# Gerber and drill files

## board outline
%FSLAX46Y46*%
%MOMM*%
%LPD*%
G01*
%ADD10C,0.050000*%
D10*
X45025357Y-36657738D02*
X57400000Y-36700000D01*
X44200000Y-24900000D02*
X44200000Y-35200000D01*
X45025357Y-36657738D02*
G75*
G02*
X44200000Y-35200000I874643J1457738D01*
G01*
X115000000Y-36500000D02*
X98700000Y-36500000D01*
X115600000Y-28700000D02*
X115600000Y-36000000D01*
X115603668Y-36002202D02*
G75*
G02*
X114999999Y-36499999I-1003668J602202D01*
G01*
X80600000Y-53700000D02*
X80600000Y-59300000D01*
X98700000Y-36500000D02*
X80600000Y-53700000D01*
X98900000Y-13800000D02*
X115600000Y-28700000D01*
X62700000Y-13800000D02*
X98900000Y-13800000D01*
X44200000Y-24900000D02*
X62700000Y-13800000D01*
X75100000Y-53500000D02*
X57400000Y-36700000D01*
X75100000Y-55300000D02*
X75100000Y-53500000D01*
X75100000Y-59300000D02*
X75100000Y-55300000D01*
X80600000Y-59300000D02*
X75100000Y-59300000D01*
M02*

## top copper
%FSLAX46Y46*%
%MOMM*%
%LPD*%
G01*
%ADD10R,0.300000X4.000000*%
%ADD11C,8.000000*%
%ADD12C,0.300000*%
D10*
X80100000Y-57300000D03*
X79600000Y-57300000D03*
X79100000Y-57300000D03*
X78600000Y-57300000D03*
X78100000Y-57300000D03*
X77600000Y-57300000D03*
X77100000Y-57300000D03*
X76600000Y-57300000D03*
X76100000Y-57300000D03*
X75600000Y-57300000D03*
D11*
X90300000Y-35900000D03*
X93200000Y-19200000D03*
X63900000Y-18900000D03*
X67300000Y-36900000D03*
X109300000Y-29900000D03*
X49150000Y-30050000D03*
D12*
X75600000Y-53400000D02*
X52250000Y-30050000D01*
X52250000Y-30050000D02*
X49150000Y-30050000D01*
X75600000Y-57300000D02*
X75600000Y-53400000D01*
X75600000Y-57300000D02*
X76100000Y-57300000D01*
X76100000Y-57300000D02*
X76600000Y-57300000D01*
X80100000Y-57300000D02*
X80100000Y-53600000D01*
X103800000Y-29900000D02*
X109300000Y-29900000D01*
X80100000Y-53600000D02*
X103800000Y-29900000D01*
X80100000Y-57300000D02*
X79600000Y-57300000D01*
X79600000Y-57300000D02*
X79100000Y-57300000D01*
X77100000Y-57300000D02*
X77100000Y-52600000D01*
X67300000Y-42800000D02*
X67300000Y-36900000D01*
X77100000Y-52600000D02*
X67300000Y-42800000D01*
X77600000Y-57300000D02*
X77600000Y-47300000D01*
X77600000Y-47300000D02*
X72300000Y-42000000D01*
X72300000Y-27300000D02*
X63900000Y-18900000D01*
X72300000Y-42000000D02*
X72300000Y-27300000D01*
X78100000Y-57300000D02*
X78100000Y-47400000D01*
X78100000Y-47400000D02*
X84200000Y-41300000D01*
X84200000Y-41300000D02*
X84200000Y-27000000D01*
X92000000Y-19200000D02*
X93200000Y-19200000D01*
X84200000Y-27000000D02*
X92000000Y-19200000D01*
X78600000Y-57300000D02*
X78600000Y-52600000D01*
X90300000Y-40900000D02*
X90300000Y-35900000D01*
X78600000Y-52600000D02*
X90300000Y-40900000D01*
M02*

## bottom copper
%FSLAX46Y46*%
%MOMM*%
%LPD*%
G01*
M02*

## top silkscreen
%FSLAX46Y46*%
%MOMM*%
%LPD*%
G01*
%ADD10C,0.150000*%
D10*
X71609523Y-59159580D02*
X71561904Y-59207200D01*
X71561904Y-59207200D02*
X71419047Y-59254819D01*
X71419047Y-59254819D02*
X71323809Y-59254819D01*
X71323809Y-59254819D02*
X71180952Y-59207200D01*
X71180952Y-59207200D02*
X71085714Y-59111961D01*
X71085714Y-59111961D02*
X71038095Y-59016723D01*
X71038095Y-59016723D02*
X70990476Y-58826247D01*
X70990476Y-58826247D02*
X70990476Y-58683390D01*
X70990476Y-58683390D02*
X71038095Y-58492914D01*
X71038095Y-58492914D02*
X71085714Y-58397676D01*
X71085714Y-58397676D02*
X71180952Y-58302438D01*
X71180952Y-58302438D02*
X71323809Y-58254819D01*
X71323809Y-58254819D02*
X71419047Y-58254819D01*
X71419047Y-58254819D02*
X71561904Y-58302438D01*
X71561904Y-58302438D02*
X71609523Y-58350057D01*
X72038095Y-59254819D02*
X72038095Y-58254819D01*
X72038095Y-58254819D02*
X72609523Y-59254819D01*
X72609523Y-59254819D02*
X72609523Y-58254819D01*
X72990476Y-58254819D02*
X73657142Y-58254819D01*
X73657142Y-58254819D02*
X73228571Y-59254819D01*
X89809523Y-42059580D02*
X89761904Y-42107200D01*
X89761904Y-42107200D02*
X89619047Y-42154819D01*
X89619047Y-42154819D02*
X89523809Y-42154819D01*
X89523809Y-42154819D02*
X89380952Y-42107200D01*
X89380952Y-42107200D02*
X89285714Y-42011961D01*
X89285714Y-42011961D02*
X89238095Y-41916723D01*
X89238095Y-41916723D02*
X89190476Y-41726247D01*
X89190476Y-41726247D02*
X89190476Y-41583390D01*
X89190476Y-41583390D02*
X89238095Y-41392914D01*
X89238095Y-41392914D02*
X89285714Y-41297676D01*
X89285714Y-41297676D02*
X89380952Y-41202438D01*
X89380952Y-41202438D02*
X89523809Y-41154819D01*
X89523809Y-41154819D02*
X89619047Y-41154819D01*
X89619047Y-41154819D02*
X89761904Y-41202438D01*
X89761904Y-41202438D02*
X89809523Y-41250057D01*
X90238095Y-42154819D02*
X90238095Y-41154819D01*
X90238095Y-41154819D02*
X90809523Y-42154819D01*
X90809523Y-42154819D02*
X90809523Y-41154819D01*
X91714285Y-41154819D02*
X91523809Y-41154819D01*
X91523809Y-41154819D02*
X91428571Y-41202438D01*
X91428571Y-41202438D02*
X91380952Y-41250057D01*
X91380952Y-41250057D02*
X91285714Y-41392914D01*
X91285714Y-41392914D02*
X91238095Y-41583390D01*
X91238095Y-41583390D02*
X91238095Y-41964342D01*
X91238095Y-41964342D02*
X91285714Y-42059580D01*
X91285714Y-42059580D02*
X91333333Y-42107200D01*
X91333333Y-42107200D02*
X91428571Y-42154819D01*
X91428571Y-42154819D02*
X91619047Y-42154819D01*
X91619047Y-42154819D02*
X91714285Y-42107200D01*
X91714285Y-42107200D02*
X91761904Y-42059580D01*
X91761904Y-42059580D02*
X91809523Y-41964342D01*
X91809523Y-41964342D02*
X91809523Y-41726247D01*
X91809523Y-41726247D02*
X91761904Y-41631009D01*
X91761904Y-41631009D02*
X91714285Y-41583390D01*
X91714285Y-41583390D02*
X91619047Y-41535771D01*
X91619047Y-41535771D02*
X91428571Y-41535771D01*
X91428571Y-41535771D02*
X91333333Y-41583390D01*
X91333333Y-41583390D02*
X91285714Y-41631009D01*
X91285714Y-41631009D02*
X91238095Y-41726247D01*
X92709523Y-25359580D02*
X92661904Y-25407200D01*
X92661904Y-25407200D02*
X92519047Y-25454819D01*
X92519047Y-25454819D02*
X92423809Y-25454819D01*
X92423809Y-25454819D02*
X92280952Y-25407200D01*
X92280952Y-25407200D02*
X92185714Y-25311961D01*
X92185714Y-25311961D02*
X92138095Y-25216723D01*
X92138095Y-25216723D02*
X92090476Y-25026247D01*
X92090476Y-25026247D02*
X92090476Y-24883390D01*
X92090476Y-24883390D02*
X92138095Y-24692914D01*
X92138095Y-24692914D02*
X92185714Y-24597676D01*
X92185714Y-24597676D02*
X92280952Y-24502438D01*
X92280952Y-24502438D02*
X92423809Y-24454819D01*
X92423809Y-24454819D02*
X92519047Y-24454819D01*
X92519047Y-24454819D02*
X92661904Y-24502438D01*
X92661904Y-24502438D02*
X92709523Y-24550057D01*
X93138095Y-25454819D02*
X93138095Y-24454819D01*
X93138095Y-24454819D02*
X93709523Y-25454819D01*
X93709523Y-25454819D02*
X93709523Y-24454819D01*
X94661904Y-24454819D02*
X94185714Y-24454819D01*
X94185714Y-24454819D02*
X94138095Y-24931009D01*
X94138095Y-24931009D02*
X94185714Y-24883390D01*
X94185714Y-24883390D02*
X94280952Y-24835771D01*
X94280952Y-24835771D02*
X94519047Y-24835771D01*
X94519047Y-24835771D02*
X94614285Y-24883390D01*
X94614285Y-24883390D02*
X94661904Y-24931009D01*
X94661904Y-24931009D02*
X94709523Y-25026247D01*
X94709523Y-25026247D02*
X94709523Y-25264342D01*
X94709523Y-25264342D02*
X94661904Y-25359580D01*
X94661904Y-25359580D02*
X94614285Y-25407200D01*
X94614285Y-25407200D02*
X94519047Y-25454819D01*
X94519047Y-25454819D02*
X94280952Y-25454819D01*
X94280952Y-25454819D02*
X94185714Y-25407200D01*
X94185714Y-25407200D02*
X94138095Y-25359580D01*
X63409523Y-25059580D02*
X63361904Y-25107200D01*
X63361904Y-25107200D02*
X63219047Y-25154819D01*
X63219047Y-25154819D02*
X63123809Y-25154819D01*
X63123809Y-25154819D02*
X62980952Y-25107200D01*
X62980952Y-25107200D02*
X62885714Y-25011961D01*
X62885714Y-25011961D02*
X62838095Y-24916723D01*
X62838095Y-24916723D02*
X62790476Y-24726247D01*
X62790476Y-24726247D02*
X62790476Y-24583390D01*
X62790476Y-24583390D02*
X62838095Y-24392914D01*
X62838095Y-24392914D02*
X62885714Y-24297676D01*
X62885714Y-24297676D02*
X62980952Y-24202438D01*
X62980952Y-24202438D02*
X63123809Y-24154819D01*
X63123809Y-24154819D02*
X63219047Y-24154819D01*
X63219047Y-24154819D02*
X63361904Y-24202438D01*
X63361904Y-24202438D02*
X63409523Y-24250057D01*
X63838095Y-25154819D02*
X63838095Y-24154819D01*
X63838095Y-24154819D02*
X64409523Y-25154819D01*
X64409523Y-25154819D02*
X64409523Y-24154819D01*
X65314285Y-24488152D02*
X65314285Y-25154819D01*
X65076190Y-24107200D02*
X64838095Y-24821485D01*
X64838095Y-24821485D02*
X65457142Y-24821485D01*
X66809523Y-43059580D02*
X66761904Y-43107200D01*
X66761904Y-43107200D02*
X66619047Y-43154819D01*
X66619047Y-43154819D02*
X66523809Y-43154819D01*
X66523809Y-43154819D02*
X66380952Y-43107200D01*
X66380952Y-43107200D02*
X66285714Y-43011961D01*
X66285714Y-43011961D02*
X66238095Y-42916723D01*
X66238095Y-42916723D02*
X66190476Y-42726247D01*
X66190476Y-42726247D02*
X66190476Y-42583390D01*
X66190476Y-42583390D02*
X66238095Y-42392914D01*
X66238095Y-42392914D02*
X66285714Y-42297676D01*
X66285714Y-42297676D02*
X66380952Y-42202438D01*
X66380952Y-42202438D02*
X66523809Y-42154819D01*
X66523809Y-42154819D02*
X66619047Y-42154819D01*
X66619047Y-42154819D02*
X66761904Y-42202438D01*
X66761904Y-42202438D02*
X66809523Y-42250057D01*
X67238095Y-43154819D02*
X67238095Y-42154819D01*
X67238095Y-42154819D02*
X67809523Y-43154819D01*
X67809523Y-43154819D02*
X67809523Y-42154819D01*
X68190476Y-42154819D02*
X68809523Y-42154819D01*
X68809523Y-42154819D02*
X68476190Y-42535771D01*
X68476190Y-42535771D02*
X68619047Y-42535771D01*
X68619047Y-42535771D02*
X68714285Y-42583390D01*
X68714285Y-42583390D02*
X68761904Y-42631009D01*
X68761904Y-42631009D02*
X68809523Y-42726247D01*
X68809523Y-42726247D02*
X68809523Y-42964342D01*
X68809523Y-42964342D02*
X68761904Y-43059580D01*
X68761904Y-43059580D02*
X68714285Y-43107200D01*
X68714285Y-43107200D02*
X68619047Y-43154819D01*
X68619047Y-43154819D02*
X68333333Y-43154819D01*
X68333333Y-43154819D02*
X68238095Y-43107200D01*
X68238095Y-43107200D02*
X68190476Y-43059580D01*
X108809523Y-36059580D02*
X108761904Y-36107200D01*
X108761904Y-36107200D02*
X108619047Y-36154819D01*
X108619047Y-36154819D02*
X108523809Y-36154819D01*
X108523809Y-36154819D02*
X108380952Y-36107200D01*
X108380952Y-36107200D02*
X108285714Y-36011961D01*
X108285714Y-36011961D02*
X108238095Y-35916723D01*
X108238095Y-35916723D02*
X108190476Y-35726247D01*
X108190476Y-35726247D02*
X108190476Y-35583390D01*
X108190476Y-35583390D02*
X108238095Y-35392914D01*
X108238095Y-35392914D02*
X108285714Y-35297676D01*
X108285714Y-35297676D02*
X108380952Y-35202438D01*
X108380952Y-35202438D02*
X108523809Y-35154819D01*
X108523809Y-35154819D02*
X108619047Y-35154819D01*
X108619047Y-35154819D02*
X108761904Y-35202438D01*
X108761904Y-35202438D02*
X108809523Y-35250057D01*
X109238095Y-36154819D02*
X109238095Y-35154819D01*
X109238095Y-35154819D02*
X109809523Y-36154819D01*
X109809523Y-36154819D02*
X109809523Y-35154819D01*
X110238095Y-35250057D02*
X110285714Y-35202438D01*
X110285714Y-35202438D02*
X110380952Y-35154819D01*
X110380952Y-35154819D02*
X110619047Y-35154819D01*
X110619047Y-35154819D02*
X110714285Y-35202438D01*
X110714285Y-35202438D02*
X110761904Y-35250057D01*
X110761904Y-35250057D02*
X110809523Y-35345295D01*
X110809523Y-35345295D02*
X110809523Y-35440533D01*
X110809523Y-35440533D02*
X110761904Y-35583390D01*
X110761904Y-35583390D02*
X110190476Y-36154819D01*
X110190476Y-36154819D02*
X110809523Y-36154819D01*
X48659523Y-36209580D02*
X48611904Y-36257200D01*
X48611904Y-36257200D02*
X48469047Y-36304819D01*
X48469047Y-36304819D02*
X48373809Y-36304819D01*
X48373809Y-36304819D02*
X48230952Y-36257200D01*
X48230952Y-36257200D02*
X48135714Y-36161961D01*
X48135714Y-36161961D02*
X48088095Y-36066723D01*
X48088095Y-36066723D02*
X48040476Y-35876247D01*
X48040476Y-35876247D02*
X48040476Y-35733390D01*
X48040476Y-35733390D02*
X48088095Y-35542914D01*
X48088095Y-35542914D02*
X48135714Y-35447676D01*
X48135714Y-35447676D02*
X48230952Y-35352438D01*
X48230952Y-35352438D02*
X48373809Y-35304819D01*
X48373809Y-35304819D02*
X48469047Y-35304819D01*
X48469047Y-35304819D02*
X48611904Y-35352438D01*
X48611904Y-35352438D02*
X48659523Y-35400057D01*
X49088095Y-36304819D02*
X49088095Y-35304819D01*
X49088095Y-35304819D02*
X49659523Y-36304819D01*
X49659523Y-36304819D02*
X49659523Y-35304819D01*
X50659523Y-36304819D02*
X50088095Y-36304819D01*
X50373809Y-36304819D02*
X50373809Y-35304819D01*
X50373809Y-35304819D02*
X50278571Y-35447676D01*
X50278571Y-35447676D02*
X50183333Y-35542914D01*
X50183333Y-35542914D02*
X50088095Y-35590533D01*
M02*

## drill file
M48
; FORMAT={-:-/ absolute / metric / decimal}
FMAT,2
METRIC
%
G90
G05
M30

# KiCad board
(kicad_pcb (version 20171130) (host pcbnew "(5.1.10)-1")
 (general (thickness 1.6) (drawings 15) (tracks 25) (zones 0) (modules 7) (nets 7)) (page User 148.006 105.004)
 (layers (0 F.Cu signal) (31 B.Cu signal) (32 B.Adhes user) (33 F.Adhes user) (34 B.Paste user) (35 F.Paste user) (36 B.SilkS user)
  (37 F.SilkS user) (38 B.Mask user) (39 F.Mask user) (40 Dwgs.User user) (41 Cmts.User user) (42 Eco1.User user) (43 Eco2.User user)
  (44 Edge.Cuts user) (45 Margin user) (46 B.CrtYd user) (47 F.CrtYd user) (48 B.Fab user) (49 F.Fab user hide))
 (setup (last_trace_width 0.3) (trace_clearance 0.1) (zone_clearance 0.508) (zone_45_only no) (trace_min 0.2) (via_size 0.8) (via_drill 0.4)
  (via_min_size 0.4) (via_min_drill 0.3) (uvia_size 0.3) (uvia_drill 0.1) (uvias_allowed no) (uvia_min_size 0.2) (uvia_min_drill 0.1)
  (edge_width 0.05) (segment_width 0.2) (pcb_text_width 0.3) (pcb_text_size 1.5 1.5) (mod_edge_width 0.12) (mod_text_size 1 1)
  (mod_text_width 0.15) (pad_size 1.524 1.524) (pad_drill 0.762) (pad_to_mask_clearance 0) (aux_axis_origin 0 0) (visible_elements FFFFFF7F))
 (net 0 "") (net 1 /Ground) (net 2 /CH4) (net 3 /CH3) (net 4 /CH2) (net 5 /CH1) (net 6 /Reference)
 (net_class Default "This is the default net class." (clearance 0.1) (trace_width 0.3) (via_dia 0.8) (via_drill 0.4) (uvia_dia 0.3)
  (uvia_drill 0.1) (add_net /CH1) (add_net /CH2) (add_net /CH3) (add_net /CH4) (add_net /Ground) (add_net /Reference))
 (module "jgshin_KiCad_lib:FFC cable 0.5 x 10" (layer F.Cu) (at 75.6 57.3)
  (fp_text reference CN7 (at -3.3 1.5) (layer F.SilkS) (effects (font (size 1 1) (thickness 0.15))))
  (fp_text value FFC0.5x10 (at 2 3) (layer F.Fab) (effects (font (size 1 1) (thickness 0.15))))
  (pad 10 smd rect (at 4.5 0) (size 0.3 4) (layers F.Cu F.Paste F.Mask) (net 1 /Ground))
  (pad 9 smd rect (at 4 0) (size 0.3 4) (layers F.Cu F.Paste F.Mask) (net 1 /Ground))
  (pad 8 smd rect (at 3.5 0) (size 0.3 4) (layers F.Cu F.Paste F.Mask) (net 1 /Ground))
  (pad 7 smd rect (at 3 0) (size 0.3 4) (layers F.Cu F.Paste F.Mask) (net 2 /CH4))
  (pad 6 smd rect (at 2.5 0) (size 0.3 4) (layers F.Cu F.Paste F.Mask) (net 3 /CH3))
  (pad 5 smd rect (at 2 0) (size 0.3 4) (layers F.Cu F.Paste F.Mask) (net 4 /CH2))
  (pad 4 smd rect (at 1.5 0) (size 0.3 4) (layers F.Cu F.Paste F.Mask) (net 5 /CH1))
  (pad 3 smd rect (at 1 0) (size 0.3 4) (layers F.Cu F.Paste F.Mask) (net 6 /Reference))
  (pad 2 smd rect (at 0.5 0) (size 0.3 4) (layers F.Cu F.Paste F.Mask) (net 6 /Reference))
  (pad 1 smd rect (at 0 0) (size 0.3 4) (layers F.Cu F.Paste F.Mask) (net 6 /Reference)))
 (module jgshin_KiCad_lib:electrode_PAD (layer F.Cu) (at 90.5 41.2)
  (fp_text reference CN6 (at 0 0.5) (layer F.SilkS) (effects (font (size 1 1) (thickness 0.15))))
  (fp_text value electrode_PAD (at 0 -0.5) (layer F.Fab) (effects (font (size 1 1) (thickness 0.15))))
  (pad 1 smd circle (at -0.2 -5.3) (size 8 8) (layers F.Cu F.Paste F.Mask) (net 2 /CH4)))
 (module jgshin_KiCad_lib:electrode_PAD (layer F.Cu) (at 93.4 24.5)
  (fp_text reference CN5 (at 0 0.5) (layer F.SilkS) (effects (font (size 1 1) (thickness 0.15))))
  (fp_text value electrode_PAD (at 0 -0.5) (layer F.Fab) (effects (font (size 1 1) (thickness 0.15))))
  (pad 1 smd circle (at -0.2 -5.3) (size 8 8) (layers F.Cu F.Paste F.Mask) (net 3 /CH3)))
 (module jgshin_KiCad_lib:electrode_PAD (layer F.Cu) (at 64.1 24.2)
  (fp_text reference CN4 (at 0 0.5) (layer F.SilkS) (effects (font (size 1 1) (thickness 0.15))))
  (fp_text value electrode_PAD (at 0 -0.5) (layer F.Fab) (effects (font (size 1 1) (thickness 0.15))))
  (pad 1 smd circle (at -0.2 -5.3) (size 8 8) (layers F.Cu F.Paste F.Mask) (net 4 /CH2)))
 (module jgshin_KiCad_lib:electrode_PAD (layer F.Cu) (at 67.5 42.2)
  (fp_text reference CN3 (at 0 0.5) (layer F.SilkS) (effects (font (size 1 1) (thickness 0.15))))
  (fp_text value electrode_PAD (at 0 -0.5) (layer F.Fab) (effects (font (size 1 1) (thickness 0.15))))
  (pad 1 smd circle (at -0.2 -5.3) (size 8 8) (layers F.Cu F.Paste F.Mask) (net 5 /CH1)))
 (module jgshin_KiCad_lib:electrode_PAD (layer F.Cu) (at 109.5 35.2)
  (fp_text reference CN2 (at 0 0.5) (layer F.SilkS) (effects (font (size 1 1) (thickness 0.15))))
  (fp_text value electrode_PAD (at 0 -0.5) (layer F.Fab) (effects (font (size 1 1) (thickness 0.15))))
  (pad 1 smd circle (at -0.2 -5.3) (size 8 8) (layers F.Cu F.Paste F.Mask) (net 1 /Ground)))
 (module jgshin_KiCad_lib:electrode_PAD (layer F.Cu) (at 49.35 35.35)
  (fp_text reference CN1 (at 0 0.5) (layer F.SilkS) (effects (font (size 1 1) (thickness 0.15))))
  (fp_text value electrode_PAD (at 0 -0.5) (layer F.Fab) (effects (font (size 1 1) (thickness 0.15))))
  (pad 1 smd circle (at -0.2 -5.3) (size 8 8) (layers F.Cu F.Paste F.Mask) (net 6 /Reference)))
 (gr_line (start 45.025357 36.657738) (end 57.4 36.7) (layer Edge.Cuts) (width 0.05))
 (gr_line (start 44.2 24.9) (end 44.2 35.2) (layer Edge.Cuts) (width 0.05))
 (gr_arc (start 45.9 35.2) (end 44.2 35.2) (angle -59.03624347) (layer Edge.Cuts) (width 0.05))
 (gr_line (start 115 36.5) (end 98.7 36.5) (layer Edge.Cuts) (width 0.05))
 (gr_line (start 115.6 28.7) (end 115.6 36) (layer Edge.Cuts) (width 0.05))
 (gr_arc (start 114.6 35.4) (end 114.999999 36.499999) (angle -39.05313695) (layer Edge.Cuts) (width 0.05))
 (gr_line (start 80.6 53.7) (end 80.6 59.3) (layer Edge.Cuts) (width 0.05))
 (gr_line (start 98.7 36.5) (end 80.6 53.7) (layer Edge.Cuts) (width 0.05))
 (gr_line (start 98.9 13.8) (end 115.6 28.7) (layer Edge.Cuts) (width 0.05))
 (gr_line (start 62.7 13.8) (end 98.9 13.8) (layer Edge.Cuts) (width 0.05))
 (gr_line (start 44.2 24.9) (end 62.7 13.8) (layer Edge.Cuts) (width 0.05))
 (gr_line (start 75.1 53.5) (end 57.4 36.7) (layer Edge.Cuts) (width 0.05))
 (gr_line (start 75.1 55.3) (end 75.1 53.5) (layer Edge.Cuts) (width 0.05))
 (gr_line (start 75.1 59.3) (end 75.1 55.3) (layer Edge.Cuts) (width 0.05))
 (gr_line (start 80.6 59.3) (end 75.1 59.3) (layer Edge.Cuts) (width 0.05))
 (segment (start 75.6 53.4) (end 52.25 30.05) (width 0.3) (layer F.Cu) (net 6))
 (segment (start 52.25 30.05) (end 49.15 30.05) (width 0.3) (layer F.Cu) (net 6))
 (segment (start 75.6 57.3) (end 75.6 53.4) (width 0.3) (layer F.Cu) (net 6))
 (segment (start 75.6 57.3) (end 76.1 57.3) (width 0.3) (layer F.Cu) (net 6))
 (segment (start 76.1 57.3) (end 76.6 57.3) (width 0.3) (layer F.Cu) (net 6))
 (segment (start 80.1 57.3) (end 80.1 53.6) (width 0.3) (layer F.Cu) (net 1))
 (segment (start 103.8 29.9) (end 109.3 29.9) (width 0.3) (layer F.Cu) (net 1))
 (segment (start 80.1 53.6) (end 103.8 29.9) (width 0.3) (layer F.Cu) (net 1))
 (segment (start 80.1 57.3) (end 79.6 57.3) (width 0.3) (layer F.Cu) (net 1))
 (segment (start 79.6 57.3) (end 79.1 57.3) (width 0.3) (layer F.Cu) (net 1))
 (segment (start 77.1 57.3) (end 77.1 52.6) (width 0.3) (layer F.Cu) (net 5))
 (segment (start 67.3 42.8) (end 67.3 36.9) (width 0.3) (layer F.Cu) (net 5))
 (segment (start 77.1 52.6) (end 67.3 42.8) (width 0.3) (layer F.Cu) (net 5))
 (segment (start 77.6 57.3) (end 77.6 47.3) (width 0.3) (layer F.Cu) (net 4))
 (segment (start 77.6 47.3) (end 72.3 42) (width 0.3) (layer F.Cu) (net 4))
 (segment (start 72.3 27.3) (end 63.9 18.9) (width 0.3) (layer F.Cu) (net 4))
 (segment (start 72.3 42) (end 72.3 27.3) (width 0.3) (layer F.Cu) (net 4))
 (segment (start 78.1 57.3) (end 78.1 47.4) (width 0.3) (layer F.Cu) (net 3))
 (segment (start 78.1 47.4) (end 84.2 41.3) (width 0.3) (layer F.Cu) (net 3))
 (segment (start 84.2 41.3) (end 84.2 27) (width 0.3) (layer F.Cu) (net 3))
 (segment (start 92 19.2) (end 93.2 19.2) (width 0.3) (layer F.Cu) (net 3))
 (segment (start 84.2 27) (end 92 19.2) (width 0.3) (layer F.Cu) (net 3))
 (segment (start 78.6 57.3) (end 78.6 52.6) (width 0.3) (layer F.Cu) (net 2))
 (segment (start 90.3 40.9) (end 90.3 35.9) (width 0.3) (layer F.Cu) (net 2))
 (segment (start 78.6 52.6) (end 90.3 40.9) (width 0.3) (layer F.Cu) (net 2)))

